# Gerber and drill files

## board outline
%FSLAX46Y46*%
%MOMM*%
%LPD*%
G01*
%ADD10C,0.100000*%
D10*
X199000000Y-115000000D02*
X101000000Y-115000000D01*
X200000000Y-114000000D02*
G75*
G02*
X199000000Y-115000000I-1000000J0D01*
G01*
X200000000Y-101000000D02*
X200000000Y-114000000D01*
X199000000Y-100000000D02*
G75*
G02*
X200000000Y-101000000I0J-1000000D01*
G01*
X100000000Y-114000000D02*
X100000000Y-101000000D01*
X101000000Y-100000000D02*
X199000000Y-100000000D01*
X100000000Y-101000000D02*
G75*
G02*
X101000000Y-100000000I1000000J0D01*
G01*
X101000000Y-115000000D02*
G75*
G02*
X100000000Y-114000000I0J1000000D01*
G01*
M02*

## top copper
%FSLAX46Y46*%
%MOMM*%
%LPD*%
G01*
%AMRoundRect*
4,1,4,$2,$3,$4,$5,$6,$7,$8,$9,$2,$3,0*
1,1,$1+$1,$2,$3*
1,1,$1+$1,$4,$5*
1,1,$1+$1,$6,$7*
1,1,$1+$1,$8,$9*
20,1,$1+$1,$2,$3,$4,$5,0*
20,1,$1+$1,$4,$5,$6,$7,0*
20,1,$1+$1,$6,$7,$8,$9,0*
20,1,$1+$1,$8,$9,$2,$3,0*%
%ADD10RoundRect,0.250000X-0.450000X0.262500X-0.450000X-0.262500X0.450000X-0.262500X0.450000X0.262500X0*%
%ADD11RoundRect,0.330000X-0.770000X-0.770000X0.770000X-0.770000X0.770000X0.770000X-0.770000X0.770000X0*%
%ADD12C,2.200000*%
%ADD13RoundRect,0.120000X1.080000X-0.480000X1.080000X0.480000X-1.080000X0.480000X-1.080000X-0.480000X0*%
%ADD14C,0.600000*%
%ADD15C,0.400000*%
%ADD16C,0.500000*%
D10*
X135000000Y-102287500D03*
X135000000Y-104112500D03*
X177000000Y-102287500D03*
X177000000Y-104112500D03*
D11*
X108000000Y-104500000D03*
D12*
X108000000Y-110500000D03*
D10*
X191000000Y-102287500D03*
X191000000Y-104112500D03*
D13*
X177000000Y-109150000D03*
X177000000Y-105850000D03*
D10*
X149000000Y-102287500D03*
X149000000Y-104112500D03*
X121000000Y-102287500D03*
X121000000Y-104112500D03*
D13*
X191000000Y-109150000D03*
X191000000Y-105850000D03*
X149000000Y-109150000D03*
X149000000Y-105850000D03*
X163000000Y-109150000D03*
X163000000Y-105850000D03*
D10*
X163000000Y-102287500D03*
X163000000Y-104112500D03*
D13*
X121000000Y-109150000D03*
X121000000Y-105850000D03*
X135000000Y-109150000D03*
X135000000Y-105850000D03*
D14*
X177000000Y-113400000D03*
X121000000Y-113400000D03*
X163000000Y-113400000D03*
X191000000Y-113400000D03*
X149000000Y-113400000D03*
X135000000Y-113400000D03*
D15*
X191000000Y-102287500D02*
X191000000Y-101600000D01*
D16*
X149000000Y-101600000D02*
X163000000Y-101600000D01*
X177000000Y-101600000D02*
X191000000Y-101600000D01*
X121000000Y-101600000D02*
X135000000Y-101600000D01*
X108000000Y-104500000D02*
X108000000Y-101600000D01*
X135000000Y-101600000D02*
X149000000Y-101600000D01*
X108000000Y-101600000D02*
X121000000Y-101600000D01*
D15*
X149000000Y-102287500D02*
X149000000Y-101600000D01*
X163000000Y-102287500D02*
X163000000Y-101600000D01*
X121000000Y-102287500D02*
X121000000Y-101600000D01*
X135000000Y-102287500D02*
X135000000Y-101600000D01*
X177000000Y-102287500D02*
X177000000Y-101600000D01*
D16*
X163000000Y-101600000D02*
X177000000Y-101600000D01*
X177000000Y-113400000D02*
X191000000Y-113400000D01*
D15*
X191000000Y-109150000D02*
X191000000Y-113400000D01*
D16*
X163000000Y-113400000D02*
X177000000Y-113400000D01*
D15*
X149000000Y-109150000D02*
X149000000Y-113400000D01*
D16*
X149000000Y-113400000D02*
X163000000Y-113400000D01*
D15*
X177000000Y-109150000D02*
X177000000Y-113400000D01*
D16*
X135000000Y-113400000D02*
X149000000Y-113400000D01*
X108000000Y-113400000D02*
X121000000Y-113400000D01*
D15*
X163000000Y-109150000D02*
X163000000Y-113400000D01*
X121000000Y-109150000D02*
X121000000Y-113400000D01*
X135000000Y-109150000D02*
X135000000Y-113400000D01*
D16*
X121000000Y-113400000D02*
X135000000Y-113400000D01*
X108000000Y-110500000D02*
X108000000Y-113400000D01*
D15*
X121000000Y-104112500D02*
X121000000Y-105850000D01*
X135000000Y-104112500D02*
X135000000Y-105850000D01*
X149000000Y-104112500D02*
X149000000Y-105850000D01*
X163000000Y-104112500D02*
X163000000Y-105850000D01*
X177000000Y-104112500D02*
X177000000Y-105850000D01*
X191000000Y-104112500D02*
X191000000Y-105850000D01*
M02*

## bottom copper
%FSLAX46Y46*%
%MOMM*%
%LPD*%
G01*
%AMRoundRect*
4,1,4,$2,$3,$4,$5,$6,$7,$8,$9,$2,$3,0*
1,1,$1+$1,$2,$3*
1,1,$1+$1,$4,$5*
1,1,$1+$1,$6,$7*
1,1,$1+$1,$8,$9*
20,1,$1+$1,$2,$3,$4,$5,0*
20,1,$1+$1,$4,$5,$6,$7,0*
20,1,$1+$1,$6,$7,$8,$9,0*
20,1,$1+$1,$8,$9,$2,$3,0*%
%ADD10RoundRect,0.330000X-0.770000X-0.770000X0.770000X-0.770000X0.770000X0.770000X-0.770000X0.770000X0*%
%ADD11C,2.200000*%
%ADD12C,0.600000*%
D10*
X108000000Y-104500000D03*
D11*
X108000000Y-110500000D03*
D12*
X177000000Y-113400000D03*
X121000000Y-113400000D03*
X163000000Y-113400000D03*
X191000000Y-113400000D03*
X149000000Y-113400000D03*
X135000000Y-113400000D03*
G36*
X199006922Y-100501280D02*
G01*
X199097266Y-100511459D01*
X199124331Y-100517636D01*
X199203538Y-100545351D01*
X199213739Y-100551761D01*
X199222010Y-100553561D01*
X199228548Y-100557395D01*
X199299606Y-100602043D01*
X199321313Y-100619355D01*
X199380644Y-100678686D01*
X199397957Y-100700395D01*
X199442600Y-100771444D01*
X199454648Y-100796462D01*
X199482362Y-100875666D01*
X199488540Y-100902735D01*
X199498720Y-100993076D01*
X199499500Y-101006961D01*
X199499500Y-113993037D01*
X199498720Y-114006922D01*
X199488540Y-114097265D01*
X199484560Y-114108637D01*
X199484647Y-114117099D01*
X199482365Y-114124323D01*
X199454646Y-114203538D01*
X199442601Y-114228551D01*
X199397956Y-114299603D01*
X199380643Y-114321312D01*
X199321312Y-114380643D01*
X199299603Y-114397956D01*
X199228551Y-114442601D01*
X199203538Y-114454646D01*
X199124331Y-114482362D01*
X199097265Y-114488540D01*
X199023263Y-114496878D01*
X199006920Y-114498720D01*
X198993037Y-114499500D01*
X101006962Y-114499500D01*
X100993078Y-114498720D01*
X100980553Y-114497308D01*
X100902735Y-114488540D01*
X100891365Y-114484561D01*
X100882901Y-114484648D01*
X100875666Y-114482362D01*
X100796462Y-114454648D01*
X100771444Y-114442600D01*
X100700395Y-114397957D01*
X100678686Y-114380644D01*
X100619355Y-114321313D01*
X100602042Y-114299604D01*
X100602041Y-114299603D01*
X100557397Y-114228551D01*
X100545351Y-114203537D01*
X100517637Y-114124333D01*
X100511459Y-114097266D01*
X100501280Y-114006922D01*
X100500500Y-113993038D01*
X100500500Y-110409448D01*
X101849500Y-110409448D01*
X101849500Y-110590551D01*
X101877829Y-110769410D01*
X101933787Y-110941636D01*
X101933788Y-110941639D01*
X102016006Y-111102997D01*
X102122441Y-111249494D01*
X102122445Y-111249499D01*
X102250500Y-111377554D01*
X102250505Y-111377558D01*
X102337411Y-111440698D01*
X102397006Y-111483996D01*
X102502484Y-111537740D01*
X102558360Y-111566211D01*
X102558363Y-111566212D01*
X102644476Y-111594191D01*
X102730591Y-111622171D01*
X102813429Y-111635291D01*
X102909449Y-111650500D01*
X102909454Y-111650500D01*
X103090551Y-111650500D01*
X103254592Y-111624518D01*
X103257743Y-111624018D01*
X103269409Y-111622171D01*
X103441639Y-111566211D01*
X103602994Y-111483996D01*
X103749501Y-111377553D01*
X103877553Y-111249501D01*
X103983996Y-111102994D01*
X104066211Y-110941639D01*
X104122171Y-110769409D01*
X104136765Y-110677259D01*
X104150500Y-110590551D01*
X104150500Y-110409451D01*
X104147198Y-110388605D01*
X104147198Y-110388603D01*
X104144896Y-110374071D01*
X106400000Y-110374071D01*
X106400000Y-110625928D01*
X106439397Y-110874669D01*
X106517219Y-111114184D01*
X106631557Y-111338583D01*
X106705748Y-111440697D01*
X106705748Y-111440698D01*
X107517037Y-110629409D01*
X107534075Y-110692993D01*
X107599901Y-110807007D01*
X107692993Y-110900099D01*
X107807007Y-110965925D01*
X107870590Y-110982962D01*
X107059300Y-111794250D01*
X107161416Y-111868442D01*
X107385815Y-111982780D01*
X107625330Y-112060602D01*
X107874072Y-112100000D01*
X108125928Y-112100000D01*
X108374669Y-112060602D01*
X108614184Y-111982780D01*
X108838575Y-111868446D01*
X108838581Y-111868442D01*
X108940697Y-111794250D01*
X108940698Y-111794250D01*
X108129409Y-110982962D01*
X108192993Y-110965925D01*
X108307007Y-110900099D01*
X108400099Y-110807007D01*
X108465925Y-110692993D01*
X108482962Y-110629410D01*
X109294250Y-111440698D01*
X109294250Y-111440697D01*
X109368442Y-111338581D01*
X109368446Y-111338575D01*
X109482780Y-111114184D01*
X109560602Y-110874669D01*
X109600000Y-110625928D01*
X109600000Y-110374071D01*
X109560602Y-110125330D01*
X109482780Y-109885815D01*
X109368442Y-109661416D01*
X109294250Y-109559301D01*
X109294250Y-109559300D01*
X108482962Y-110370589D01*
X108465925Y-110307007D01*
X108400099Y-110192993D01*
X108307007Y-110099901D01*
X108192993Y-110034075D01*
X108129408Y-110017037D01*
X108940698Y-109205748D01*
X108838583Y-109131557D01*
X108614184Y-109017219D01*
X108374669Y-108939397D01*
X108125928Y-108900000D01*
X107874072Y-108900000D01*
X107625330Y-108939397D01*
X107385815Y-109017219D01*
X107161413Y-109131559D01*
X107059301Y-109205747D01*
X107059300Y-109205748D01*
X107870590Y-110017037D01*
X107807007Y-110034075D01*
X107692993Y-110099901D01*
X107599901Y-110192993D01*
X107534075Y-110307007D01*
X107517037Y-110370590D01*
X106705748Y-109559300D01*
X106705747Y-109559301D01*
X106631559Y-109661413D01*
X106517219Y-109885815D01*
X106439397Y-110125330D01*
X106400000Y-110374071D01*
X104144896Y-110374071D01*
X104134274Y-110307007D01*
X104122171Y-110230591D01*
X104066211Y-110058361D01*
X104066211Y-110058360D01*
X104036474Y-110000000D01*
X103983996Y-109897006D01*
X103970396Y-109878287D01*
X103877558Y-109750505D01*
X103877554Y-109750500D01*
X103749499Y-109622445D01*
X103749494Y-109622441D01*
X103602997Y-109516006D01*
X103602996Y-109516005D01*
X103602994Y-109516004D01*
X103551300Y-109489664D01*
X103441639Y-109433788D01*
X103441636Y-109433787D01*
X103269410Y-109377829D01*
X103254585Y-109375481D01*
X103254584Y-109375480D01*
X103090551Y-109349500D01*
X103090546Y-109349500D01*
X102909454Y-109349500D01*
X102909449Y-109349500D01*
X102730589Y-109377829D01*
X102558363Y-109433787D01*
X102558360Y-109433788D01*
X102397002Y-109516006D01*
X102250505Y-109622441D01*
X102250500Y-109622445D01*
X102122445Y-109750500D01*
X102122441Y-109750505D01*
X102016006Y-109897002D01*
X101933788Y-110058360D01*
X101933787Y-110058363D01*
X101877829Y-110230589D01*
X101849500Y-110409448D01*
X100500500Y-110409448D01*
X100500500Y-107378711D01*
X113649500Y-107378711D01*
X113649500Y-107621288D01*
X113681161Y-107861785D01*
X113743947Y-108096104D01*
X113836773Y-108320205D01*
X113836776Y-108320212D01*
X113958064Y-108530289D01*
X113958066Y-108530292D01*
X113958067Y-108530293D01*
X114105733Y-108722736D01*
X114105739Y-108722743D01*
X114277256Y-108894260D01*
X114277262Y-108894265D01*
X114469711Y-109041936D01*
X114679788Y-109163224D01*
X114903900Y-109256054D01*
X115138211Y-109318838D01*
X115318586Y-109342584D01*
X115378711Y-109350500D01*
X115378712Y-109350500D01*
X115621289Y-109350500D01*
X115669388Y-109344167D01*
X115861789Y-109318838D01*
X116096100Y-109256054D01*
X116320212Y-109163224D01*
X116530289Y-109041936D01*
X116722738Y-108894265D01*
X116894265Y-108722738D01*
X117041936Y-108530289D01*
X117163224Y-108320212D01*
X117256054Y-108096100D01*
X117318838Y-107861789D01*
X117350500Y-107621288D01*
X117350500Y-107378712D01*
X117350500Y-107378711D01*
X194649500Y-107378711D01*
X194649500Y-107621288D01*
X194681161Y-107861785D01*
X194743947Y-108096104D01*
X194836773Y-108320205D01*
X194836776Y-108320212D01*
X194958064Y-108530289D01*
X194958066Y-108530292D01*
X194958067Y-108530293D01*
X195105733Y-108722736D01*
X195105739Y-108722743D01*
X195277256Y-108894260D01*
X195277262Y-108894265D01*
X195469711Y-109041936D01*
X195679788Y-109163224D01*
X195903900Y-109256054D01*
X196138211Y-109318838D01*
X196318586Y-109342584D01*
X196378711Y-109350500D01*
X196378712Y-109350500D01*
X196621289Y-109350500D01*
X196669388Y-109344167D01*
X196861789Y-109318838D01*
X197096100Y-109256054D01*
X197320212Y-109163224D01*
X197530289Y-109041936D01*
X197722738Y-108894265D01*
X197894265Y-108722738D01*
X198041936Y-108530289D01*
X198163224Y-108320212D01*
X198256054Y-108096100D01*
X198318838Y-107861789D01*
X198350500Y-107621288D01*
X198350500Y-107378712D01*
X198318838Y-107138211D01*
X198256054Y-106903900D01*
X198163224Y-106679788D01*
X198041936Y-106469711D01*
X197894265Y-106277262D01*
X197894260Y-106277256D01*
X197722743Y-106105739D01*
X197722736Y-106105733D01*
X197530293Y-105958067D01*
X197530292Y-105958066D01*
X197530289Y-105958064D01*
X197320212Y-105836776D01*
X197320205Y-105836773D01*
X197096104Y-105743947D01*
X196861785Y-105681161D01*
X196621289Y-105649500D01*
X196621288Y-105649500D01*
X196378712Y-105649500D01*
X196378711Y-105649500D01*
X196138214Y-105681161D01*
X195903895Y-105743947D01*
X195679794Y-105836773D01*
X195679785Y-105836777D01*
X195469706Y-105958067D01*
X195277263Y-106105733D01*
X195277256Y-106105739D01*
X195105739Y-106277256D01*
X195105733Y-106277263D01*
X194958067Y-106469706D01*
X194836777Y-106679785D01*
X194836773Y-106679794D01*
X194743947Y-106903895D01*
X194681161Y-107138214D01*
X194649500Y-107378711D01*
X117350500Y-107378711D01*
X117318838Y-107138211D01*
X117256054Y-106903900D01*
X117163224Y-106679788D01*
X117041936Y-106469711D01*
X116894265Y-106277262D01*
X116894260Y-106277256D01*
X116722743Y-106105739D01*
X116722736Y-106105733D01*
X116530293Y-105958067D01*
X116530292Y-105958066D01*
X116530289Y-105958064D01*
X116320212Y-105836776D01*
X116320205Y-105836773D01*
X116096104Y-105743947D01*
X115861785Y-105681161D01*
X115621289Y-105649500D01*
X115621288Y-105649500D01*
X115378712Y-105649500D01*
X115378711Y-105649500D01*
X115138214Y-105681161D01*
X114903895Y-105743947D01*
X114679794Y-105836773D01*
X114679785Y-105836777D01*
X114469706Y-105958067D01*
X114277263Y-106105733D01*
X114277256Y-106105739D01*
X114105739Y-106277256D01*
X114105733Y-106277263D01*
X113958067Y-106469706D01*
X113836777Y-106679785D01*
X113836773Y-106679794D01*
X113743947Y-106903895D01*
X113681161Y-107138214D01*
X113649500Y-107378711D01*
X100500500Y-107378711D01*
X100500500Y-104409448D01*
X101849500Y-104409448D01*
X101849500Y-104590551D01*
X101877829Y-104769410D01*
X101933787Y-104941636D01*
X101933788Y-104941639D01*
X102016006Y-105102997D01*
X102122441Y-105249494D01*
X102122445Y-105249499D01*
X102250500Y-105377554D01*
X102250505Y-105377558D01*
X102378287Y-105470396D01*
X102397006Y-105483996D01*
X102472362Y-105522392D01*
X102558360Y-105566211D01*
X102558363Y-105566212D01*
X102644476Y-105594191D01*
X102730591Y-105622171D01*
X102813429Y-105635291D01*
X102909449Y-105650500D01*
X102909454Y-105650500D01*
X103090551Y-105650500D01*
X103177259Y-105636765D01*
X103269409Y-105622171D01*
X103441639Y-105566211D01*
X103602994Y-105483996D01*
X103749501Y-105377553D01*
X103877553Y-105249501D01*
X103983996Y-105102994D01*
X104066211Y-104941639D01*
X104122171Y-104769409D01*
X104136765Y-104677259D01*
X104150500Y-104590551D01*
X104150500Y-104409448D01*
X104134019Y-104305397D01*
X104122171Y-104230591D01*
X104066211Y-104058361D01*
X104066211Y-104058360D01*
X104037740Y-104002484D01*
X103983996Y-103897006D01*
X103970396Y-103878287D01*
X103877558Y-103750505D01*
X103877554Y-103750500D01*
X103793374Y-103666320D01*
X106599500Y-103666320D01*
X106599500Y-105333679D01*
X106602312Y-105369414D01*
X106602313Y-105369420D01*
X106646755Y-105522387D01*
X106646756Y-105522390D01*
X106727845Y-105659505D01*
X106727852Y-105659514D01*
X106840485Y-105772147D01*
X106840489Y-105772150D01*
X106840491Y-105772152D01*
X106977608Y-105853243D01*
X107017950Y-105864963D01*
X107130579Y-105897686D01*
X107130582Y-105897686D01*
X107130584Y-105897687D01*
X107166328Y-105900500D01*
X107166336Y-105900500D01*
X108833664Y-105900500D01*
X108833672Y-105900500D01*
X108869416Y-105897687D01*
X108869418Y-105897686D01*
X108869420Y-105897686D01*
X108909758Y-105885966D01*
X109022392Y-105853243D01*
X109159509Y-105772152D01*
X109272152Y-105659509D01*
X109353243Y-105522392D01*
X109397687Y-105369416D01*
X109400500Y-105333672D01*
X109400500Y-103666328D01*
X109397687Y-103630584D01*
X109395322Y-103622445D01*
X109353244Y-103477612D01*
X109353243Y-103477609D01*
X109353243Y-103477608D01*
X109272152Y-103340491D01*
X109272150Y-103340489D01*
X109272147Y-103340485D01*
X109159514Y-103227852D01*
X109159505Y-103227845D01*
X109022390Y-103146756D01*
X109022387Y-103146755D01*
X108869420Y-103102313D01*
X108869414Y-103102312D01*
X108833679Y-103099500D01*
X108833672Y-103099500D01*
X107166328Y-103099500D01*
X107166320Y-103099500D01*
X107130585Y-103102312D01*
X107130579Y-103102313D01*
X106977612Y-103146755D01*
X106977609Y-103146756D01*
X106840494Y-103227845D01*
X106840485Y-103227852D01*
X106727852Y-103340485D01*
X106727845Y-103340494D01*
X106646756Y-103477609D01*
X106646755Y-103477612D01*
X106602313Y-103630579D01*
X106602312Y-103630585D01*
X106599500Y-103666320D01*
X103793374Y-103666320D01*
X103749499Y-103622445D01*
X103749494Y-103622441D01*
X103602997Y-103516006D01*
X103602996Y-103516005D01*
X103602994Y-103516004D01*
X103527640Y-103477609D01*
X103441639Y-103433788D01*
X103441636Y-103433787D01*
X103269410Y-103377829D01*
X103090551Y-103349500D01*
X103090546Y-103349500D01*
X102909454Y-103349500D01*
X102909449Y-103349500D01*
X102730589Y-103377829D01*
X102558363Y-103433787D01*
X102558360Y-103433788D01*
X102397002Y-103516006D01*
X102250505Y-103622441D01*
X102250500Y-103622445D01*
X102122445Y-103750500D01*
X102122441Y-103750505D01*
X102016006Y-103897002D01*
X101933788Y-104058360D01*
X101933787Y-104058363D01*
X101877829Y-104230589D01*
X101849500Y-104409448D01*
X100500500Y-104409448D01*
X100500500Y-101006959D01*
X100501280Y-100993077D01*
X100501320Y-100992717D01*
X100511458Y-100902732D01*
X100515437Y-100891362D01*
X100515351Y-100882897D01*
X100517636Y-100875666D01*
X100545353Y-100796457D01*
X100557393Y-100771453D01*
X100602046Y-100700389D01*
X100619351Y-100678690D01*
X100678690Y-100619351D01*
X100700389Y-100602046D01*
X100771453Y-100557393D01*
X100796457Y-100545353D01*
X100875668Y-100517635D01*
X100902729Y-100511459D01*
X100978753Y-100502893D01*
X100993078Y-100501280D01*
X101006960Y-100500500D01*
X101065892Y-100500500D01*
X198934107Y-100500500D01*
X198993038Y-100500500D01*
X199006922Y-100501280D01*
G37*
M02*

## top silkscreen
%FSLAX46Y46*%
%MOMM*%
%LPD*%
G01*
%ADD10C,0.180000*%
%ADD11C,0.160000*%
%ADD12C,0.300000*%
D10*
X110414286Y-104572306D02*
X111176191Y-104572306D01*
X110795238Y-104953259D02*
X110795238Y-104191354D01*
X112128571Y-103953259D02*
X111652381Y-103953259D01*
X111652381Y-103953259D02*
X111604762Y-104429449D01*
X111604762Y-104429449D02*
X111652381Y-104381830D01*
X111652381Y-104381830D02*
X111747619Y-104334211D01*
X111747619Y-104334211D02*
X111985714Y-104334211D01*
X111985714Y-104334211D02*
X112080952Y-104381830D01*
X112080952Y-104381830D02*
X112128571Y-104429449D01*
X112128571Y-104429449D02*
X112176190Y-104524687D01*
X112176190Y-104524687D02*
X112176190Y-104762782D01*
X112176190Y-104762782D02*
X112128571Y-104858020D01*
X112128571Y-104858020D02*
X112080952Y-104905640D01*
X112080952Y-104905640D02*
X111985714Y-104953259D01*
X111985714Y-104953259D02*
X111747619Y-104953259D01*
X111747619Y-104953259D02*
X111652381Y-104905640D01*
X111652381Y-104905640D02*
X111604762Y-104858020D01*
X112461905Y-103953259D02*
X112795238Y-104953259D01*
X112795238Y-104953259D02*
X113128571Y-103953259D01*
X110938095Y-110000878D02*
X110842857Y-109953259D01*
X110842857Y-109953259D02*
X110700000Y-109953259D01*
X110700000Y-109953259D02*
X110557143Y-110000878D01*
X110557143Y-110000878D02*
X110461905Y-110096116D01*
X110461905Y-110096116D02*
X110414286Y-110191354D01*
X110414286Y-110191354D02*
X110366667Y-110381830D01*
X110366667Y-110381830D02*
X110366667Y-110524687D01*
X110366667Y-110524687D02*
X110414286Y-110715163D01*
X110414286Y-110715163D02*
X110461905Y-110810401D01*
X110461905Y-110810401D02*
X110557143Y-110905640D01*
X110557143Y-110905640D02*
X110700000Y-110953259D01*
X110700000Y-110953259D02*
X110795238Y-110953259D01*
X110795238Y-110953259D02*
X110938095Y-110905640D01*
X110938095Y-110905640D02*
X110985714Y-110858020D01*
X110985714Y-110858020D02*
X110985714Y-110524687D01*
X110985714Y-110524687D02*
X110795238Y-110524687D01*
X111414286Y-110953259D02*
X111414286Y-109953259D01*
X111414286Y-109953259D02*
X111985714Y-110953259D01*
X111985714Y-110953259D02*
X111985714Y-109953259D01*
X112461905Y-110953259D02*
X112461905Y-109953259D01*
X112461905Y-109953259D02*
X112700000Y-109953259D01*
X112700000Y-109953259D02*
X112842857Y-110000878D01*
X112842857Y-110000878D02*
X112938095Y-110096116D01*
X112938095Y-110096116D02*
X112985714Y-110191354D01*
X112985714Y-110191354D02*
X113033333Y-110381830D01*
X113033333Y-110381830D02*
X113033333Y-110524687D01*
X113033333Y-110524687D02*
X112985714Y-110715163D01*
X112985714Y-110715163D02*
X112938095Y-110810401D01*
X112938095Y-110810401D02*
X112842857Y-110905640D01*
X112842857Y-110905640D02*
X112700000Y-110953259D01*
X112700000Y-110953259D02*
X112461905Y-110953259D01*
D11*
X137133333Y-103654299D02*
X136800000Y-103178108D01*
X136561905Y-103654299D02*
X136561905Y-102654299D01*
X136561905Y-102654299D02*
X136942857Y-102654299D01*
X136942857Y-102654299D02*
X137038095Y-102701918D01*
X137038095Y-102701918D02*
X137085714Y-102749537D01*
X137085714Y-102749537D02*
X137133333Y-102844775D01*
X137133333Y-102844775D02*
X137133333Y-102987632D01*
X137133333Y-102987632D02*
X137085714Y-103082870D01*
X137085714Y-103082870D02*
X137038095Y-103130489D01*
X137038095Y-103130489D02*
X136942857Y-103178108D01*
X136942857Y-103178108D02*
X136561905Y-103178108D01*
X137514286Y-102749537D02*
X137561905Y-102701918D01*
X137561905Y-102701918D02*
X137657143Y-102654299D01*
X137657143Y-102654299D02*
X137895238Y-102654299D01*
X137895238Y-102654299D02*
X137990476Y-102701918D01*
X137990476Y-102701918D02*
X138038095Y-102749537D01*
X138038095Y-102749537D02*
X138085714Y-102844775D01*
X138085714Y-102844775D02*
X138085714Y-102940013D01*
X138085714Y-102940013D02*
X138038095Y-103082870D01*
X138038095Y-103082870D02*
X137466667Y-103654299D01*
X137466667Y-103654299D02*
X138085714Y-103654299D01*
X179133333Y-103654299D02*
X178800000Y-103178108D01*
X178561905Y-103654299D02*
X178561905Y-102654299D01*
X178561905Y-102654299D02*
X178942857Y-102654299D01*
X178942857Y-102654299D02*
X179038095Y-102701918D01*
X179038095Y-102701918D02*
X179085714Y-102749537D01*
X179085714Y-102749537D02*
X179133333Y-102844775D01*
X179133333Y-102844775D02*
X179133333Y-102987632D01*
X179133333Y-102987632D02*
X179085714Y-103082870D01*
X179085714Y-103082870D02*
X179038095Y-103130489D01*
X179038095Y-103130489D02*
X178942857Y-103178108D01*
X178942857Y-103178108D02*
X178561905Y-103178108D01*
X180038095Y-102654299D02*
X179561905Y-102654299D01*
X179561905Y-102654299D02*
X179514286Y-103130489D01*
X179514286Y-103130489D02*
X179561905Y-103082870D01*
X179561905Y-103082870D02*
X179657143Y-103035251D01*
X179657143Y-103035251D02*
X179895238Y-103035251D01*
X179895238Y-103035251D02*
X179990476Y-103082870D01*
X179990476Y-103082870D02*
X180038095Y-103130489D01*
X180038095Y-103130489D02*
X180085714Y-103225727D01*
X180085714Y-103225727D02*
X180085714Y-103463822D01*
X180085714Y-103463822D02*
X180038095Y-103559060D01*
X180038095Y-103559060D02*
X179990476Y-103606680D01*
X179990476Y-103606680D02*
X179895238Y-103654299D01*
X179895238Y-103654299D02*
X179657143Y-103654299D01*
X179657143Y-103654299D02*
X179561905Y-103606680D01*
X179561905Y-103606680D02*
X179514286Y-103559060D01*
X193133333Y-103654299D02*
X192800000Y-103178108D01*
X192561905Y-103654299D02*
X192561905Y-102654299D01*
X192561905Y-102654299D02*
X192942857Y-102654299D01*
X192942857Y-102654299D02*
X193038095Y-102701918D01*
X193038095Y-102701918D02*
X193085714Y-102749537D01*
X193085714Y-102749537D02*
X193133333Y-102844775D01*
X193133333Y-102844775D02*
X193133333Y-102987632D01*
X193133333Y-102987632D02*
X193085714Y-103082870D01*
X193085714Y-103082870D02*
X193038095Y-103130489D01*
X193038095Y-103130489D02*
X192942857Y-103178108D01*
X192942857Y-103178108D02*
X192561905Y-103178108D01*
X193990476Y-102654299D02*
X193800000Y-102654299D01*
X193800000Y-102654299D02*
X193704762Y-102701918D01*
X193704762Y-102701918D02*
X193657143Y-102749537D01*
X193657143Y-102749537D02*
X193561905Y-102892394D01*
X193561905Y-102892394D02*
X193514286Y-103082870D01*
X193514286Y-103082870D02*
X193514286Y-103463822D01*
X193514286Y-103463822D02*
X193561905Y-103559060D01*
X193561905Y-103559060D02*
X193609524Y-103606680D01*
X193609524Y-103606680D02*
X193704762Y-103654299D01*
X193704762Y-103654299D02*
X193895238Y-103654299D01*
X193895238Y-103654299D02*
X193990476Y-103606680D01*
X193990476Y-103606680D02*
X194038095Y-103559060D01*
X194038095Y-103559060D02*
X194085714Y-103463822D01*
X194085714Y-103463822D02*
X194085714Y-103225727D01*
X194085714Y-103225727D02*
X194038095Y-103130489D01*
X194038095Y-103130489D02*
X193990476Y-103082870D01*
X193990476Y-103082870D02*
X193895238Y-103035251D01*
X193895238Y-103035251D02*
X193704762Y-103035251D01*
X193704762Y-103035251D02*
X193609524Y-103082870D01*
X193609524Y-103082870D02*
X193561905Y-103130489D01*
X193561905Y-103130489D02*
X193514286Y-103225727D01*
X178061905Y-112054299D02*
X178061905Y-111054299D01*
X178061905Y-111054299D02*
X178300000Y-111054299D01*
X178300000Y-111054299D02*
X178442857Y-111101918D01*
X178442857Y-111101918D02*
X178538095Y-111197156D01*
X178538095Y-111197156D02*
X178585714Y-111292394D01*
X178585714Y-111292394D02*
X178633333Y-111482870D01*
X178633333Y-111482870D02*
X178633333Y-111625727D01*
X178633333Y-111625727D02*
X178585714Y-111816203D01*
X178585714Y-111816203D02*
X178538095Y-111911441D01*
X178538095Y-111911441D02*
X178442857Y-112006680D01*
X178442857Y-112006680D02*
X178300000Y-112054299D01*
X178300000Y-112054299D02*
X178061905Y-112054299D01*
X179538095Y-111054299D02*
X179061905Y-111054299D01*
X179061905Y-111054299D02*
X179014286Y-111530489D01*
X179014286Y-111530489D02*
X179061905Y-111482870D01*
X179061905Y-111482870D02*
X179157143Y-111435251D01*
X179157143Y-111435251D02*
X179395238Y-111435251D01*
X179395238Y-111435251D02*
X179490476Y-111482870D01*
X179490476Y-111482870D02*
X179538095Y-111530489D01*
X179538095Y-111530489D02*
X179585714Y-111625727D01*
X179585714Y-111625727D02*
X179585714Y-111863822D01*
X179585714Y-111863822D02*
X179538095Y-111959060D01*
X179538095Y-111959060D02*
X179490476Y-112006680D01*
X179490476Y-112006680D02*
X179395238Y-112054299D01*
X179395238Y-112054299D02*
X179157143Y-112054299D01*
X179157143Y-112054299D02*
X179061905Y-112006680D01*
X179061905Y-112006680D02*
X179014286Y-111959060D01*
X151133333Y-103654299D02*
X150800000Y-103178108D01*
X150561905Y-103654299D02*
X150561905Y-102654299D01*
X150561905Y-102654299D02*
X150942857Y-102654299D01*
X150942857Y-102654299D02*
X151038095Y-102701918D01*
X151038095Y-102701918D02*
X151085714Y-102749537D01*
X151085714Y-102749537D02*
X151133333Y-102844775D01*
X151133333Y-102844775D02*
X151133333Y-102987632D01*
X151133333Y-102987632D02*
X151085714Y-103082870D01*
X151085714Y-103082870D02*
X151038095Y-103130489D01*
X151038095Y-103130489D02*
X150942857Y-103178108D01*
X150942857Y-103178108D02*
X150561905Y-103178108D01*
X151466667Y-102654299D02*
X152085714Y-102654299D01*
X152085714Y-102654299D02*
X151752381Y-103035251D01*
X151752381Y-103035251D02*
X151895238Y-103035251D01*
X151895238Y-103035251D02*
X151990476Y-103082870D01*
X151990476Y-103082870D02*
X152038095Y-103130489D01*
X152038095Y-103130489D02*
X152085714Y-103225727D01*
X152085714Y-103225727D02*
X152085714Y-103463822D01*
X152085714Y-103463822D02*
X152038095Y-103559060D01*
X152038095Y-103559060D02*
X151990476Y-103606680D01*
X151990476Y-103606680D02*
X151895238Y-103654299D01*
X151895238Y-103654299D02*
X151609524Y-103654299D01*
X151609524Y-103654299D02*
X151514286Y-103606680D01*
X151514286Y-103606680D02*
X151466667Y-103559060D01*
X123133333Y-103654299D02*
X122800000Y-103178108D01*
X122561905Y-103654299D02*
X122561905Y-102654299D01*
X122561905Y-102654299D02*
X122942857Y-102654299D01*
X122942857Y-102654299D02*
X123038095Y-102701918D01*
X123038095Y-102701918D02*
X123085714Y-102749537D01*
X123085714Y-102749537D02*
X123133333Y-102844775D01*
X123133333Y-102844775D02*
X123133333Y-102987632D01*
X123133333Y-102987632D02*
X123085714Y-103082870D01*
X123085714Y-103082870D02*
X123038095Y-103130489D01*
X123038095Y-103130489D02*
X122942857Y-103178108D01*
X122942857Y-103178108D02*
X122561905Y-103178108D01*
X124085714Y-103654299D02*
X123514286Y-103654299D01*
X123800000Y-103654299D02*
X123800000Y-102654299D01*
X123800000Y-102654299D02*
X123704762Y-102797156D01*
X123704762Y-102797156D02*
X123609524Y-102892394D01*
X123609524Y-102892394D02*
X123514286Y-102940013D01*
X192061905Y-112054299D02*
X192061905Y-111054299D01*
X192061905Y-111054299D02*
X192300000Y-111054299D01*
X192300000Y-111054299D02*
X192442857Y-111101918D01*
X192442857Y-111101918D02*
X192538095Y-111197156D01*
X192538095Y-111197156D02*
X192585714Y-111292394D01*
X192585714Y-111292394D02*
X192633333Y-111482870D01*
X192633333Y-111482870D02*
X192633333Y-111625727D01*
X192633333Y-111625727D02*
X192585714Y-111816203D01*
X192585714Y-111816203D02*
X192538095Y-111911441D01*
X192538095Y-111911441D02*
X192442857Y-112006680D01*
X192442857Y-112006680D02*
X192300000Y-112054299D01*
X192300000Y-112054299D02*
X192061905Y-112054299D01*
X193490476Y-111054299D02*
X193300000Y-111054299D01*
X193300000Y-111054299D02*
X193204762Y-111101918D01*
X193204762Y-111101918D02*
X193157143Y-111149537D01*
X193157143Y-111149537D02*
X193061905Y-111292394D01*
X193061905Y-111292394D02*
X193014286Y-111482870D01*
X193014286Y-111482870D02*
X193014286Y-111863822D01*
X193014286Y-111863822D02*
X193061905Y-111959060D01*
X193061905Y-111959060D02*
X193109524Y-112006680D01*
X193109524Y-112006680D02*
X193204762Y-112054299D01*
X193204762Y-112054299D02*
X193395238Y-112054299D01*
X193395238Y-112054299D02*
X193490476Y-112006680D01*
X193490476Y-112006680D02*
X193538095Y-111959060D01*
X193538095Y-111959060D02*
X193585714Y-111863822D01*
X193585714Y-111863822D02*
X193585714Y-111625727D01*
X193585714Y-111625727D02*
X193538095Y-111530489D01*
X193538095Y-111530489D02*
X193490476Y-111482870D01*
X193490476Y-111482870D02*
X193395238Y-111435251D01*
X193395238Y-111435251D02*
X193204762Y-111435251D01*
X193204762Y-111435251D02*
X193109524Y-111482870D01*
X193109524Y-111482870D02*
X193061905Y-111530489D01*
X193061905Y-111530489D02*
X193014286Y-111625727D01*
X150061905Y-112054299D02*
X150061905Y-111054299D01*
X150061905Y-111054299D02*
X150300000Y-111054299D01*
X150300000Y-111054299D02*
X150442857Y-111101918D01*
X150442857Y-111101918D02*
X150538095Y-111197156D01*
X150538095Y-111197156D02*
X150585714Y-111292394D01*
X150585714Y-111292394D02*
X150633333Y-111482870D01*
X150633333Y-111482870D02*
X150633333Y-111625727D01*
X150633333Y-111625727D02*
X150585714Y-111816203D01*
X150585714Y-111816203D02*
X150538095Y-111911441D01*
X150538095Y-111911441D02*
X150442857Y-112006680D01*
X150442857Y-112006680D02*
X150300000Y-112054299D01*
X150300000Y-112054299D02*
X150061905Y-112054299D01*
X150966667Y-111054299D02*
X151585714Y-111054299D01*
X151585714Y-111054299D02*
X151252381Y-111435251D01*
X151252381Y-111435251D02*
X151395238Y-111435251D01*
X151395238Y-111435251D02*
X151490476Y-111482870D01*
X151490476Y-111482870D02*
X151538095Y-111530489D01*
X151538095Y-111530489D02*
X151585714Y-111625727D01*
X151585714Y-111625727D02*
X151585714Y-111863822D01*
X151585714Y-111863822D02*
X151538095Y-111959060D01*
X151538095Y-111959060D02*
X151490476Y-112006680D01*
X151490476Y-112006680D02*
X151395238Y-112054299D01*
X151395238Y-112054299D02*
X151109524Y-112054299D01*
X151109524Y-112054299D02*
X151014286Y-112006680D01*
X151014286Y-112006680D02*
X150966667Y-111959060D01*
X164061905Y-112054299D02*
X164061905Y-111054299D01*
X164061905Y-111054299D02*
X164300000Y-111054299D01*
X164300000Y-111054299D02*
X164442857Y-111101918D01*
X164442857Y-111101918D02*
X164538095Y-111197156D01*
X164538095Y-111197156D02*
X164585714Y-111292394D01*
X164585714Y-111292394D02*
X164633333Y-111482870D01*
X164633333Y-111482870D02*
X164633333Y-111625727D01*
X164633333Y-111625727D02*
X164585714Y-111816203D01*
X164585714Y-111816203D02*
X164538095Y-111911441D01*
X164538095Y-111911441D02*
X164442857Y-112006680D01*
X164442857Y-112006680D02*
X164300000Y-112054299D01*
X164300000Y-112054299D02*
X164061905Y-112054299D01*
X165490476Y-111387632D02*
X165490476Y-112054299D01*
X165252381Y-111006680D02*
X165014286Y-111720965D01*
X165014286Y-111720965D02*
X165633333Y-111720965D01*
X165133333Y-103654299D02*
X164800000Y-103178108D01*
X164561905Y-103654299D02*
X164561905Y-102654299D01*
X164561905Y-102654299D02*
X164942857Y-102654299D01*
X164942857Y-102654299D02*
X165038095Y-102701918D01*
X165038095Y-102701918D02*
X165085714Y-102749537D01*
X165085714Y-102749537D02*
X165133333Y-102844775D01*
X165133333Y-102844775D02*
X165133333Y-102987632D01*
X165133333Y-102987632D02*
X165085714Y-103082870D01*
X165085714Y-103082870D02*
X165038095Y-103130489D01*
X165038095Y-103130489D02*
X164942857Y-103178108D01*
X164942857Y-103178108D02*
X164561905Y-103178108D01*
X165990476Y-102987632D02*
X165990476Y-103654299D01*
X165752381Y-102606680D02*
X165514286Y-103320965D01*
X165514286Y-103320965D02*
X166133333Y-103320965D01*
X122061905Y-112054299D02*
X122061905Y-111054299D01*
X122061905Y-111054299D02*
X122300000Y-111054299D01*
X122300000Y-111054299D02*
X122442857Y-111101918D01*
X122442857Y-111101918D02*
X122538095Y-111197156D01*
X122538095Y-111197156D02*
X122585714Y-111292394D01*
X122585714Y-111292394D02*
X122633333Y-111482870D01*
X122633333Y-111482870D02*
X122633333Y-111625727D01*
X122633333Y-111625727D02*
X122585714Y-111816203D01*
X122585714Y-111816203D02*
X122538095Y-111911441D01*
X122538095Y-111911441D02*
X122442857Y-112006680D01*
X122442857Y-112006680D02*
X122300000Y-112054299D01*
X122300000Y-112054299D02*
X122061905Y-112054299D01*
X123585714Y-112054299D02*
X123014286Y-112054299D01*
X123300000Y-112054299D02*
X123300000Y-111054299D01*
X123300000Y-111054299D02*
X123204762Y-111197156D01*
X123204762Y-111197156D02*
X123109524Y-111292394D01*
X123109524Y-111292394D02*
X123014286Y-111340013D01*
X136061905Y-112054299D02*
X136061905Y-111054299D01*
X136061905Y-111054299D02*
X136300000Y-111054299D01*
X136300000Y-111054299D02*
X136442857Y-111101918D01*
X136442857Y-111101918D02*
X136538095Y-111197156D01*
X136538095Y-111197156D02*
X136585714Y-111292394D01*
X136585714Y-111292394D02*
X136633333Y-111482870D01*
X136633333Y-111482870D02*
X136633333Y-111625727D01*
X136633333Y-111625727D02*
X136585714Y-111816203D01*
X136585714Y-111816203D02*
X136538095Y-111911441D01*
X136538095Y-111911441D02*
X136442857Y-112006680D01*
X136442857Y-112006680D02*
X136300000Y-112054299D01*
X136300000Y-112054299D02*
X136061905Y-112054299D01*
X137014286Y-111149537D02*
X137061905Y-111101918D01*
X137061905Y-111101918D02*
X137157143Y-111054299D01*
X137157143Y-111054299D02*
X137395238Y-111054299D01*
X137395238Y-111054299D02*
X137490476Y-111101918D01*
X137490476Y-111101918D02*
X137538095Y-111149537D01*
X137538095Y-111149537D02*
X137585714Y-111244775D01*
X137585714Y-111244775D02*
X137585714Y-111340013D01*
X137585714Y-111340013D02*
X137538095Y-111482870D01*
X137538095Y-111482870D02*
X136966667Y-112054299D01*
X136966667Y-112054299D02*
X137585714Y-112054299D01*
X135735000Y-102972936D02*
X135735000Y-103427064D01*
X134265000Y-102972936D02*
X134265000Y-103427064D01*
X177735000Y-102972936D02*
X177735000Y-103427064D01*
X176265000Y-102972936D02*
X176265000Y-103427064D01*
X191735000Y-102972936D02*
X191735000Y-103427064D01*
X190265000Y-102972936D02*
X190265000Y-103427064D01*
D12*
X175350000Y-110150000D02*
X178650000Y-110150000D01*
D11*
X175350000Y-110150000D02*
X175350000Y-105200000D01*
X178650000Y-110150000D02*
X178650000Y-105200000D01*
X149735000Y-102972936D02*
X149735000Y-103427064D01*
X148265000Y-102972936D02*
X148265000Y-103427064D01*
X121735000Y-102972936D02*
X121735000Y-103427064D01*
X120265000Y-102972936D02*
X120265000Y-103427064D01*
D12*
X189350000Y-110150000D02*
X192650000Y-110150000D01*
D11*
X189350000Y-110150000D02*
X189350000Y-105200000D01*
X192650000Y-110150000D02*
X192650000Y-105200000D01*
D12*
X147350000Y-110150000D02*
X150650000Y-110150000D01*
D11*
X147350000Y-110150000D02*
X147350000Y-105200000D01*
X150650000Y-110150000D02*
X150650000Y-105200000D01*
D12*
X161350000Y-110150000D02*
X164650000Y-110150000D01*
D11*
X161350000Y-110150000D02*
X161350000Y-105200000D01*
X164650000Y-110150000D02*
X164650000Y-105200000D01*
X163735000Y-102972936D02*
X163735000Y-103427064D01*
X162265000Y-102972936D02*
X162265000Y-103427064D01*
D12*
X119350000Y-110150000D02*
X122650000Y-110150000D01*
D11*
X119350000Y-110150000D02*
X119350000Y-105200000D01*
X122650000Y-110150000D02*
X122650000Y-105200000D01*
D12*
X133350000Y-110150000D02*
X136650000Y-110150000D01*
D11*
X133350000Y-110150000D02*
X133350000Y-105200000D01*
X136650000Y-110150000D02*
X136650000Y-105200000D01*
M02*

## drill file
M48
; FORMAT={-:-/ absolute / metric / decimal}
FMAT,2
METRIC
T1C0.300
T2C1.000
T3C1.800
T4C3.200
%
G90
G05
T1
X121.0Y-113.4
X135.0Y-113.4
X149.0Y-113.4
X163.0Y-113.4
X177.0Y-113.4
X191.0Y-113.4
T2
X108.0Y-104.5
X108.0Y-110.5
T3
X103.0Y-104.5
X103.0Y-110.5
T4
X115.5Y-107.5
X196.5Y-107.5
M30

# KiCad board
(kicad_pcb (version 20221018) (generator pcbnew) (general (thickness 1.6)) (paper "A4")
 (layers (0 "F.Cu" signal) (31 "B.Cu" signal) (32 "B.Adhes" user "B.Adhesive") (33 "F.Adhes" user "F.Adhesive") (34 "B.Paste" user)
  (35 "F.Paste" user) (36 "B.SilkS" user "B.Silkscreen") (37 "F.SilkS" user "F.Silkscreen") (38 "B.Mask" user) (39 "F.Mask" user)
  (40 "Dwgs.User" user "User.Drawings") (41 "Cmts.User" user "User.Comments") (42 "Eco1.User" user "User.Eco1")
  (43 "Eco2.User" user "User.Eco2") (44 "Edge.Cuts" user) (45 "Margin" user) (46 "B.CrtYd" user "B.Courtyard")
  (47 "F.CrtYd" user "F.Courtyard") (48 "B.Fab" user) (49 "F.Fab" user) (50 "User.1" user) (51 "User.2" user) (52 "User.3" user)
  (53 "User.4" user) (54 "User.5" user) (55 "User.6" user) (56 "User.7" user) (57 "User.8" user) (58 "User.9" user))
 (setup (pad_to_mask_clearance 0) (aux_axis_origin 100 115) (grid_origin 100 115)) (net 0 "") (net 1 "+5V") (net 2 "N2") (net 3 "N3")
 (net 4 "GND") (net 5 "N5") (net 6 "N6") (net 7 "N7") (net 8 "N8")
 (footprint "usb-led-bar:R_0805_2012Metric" (layer "F.Cu") (at 135 103.2 -90)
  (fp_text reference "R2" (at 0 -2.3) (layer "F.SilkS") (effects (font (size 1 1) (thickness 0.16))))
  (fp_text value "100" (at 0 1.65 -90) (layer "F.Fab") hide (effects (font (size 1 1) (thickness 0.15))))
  (fp_line (start -0.227064 -0.735) (end 0.227064 -0.735) (stroke (width 0.16) (type solid)) (layer "F.SilkS"))
  (fp_line (start -0.227064 0.735) (end 0.227064 0.735) (stroke (width 0.16) (type solid)) (layer "F.SilkS"))
  (pad "1" smd roundrect (at -0.9125 0 270) (size 1.025 1.4) (layers "F.Cu" "F.Paste" "F.Mask") (roundrect_rratio 0.243902) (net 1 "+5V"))
  (pad "2" smd roundrect (at 0.9125 0 270) (size 1.025 1.4) (layers "F.Cu" "F.Paste" "F.Mask") (roundrect_rratio 0.243902) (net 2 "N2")))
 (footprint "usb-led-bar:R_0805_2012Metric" (layer "F.Cu") (at 177 103.2 -90)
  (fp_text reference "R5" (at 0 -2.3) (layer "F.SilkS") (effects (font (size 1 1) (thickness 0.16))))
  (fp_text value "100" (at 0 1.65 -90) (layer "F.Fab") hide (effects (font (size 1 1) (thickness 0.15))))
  (fp_line (start -0.227064 -0.735) (end 0.227064 -0.735) (stroke (width 0.16) (type solid)) (layer "F.SilkS"))
  (fp_line (start -0.227064 0.735) (end 0.227064 0.735) (stroke (width 0.16) (type solid)) (layer "F.SilkS"))
  (pad "1" smd roundrect (at -0.9125 0 270) (size 1.025 1.4) (layers "F.Cu" "F.Paste" "F.Mask") (roundrect_rratio 0.243902) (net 1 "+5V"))
  (pad "2" smd roundrect (at 0.9125 0 270) (size 1.025 1.4) (layers "F.Cu" "F.Paste" "F.Mask") (roundrect_rratio 0.243902) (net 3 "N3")))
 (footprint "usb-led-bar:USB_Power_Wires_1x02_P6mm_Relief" (layer "F.Cu") (at 108 107.5)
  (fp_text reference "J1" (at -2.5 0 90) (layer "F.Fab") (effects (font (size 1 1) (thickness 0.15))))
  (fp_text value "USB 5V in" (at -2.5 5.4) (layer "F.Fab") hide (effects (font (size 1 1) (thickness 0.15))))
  (pad "" np_thru_hole circle (at -5 -3) (size 1.8 1.8) (drill 1.8) (layers "*.Cu" "*.Mask"))
  (pad "" np_thru_hole circle (at -5 3) (size 1.8 1.8) (drill 1.8) (layers "*.Cu" "*.Mask"))
  (pad "1" thru_hole roundrect (at 0 -3) (size 2.2 2.2) (drill 1) (layers "*.Cu" "*.Mask") (roundrect_rratio 0.15) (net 1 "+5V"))
  (pad "2" thru_hole circle (at 0 3) (size 2.2 2.2) (drill 1) (layers "*.Cu" "*.Mask") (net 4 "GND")))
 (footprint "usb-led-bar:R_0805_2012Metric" (layer "F.Cu") (at 191 103.2 -90)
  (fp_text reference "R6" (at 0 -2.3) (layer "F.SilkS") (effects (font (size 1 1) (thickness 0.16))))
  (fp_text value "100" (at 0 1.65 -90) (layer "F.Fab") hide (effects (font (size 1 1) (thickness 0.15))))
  (fp_line (start -0.227064 -0.735) (end 0.227064 -0.735) (stroke (width 0.16) (type solid)) (layer "F.SilkS"))
  (fp_line (start -0.227064 0.735) (end 0.227064 0.735) (stroke (width 0.16) (type solid)) (layer "F.SilkS"))
  (pad "1" smd roundrect (at -0.9125 0 270) (size 1.025 1.4) (layers "F.Cu" "F.Paste" "F.Mask") (roundrect_rratio 0.243902) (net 1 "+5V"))
  (pad "2" smd roundrect (at 0.9125 0 270) (size 1.025 1.4) (layers "F.Cu" "F.Paste" "F.Mask") (roundrect_rratio 0.243902) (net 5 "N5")))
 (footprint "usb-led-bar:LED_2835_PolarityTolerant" (layer "F.Cu") (at 177 107.5 90)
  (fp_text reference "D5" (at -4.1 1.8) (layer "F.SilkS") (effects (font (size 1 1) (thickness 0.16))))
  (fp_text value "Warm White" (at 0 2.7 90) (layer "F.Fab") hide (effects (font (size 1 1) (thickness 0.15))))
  (fp_line (start -2.65 -1.65) (end -2.65 1.65) (stroke (width 0.3) (type solid)) (layer "F.SilkS"))
  (fp_line (start -2.65 -1.65) (end 2.3 -1.65) (stroke (width 0.16) (type solid)) (layer "F.SilkS"))
  (fp_line (start -2.65 1.65) (end 2.3 1.65) (stroke (width 0.16) (type solid)) (layer "F.SilkS"))
  (pad "1" smd roundrect (at -1.65 0 90) (size 1.2 2.4) (layers "F.Cu" "F.Paste" "F.Mask") (roundrect_rratio 0.1) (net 4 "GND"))
  (pad "2" smd roundrect (at 1.65 0 90) (size 1.2 2.4) (layers "F.Cu" "F.Paste" "F.Mask") (roundrect_rratio 0.1) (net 3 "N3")))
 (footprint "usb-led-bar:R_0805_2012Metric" (layer "F.Cu") (at 149 103.2 -90)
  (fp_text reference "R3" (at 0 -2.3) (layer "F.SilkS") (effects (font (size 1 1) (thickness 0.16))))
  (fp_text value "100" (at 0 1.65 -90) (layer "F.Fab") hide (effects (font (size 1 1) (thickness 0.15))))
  (fp_line (start -0.227064 -0.735) (end 0.227064 -0.735) (stroke (width 0.16) (type solid)) (layer "F.SilkS"))
  (fp_line (start -0.227064 0.735) (end 0.227064 0.735) (stroke (width 0.16) (type solid)) (layer "F.SilkS"))
  (pad "1" smd roundrect (at -0.9125 0 270) (size 1.025 1.4) (layers "F.Cu" "F.Paste" "F.Mask") (roundrect_rratio 0.243902) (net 1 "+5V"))
  (pad "2" smd roundrect (at 0.9125 0 270) (size 1.025 1.4) (layers "F.Cu" "F.Paste" "F.Mask") (roundrect_rratio 0.243902) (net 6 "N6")))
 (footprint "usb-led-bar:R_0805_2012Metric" (layer "F.Cu") (at 121 103.2 -90)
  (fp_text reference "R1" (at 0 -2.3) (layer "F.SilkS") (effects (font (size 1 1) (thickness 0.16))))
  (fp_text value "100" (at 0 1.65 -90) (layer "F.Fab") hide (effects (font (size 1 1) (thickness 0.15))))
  (fp_line (start -0.227064 -0.735) (end 0.227064 -0.735) (stroke (width 0.16) (type solid)) (layer "F.SilkS"))
  (fp_line (start -0.227064 0.735) (end 0.227064 0.735) (stroke (width 0.16) (type solid)) (layer "F.SilkS"))
  (pad "1" smd roundrect (at -0.9125 0 270) (size 1.025 1.4) (layers "F.Cu" "F.Paste" "F.Mask") (roundrect_rratio 0.243902) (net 1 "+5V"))
  (pad "2" smd roundrect (at 0.9125 0 270) (size 1.025 1.4) (layers "F.Cu" "F.Paste" "F.Mask") (roundrect_rratio 0.243902) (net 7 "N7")))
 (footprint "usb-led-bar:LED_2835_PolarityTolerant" (layer "F.Cu") (at 191 107.5 90)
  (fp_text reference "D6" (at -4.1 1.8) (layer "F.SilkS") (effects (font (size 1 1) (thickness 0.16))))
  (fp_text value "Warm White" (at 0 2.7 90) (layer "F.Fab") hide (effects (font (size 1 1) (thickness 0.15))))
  (fp_line (start -2.65 -1.65) (end -2.65 1.65) (stroke (width 0.3) (type solid)) (layer "F.SilkS"))
  (fp_line (start -2.65 -1.65) (end 2.3 -1.65) (stroke (width 0.16) (type solid)) (layer "F.SilkS"))
  (fp_line (start -2.65 1.65) (end 2.3 1.65) (stroke (width 0.16) (type solid)) (layer "F.SilkS"))
  (pad "1" smd roundrect (at -1.65 0 90) (size 1.2 2.4) (layers "F.Cu" "F.Paste" "F.Mask") (roundrect_rratio 0.1) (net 4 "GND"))
  (pad "2" smd roundrect (at 1.65 0 90) (size 1.2 2.4) (layers "F.Cu" "F.Paste" "F.Mask") (roundrect_rratio 0.1) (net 5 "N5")))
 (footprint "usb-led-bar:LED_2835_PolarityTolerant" (layer "F.Cu") (at 149 107.5 90)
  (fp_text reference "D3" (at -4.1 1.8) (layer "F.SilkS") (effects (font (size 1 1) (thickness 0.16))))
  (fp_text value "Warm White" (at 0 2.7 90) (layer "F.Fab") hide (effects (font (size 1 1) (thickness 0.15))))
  (fp_line (start -2.65 -1.65) (end -2.65 1.65) (stroke (width 0.3) (type solid)) (layer "F.SilkS"))
  (fp_line (start -2.65 -1.65) (end 2.3 -1.65) (stroke (width 0.16) (type solid)) (layer "F.SilkS"))
  (fp_line (start -2.65 1.65) (end 2.3 1.65) (stroke (width 0.16) (type solid)) (layer "F.SilkS"))
  (pad "1" smd roundrect (at -1.65 0 90) (size 1.2 2.4) (layers "F.Cu" "F.Paste" "F.Mask") (roundrect_rratio 0.1) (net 4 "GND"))
  (pad "2" smd roundrect (at 1.65 0 90) (size 1.2 2.4) (layers "F.Cu" "F.Paste" "F.Mask") (roundrect_rratio 0.1) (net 6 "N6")))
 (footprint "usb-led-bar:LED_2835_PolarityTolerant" (layer "F.Cu") (at 163 107.5 90)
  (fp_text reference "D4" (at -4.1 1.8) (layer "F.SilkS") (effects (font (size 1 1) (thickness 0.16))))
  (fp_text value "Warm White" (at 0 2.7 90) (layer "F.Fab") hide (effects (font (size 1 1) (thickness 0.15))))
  (fp_line (start -2.65 -1.65) (end -2.65 1.65) (stroke (width 0.3) (type solid)) (layer "F.SilkS"))
  (fp_line (start -2.65 -1.65) (end 2.3 -1.65) (stroke (width 0.16) (type solid)) (layer "F.SilkS"))
  (fp_line (start -2.65 1.65) (end 2.3 1.65) (stroke (width 0.16) (type solid)) (layer "F.SilkS"))
  (pad "1" smd roundrect (at -1.65 0 90) (size 1.2 2.4) (layers "F.Cu" "F.Paste" "F.Mask") (roundrect_rratio 0.1) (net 4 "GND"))
  (pad "2" smd roundrect (at 1.65 0 90) (size 1.2 2.4) (layers "F.Cu" "F.Paste" "F.Mask") (roundrect_rratio 0.1) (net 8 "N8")))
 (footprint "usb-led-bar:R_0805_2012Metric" (layer "F.Cu") (at 163 103.2 -90)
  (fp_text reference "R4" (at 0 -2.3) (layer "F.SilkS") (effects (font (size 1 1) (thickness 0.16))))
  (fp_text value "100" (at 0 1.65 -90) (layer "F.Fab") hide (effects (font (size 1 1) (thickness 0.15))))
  (fp_line (start -0.227064 -0.735) (end 0.227064 -0.735) (stroke (width 0.16) (type solid)) (layer "F.SilkS"))
  (fp_line (start -0.227064 0.735) (end 0.227064 0.735) (stroke (width 0.16) (type solid)) (layer "F.SilkS"))
  (pad "1" smd roundrect (at -0.9125 0 270) (size 1.025 1.4) (layers "F.Cu" "F.Paste" "F.Mask") (roundrect_rratio 0.243902) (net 1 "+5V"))
  (pad "2" smd roundrect (at 0.9125 0 270) (size 1.025 1.4) (layers "F.Cu" "F.Paste" "F.Mask") (roundrect_rratio 0.243902) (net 8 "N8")))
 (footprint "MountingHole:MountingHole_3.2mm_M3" (layer "F.Cu") (at 196.5 107.5)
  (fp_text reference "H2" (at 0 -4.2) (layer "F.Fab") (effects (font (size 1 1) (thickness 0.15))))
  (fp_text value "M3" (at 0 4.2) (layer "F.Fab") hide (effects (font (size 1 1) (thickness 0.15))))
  (pad "" np_thru_hole circle (at 0 0) (size 3.2 3.2) (drill 3.2) (layers "*.Cu" "*.Mask")))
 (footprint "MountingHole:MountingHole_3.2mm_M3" (layer "F.Cu") (at 115.5 107.5)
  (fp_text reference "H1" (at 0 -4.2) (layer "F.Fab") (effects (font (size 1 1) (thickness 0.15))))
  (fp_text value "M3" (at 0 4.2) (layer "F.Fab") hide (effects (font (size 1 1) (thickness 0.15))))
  (pad "" np_thru_hole circle (at 0 0) (size 3.2 3.2) (drill 3.2) (layers "*.Cu" "*.Mask")))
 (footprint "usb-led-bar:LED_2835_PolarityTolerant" (layer "F.Cu") (at 121 107.5 90)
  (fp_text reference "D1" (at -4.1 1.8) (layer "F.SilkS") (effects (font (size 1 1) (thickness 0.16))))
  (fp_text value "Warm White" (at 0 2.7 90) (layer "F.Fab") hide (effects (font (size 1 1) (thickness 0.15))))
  (fp_line (start -2.65 -1.65) (end -2.65 1.65) (stroke (width 0.3) (type solid)) (layer "F.SilkS"))
  (fp_line (start -2.65 -1.65) (end 2.3 -1.65) (stroke (width 0.16) (type solid)) (layer "F.SilkS"))
  (fp_line (start -2.65 1.65) (end 2.3 1.65) (stroke (width 0.16) (type solid)) (layer "F.SilkS"))
  (pad "1" smd roundrect (at -1.65 0 90) (size 1.2 2.4) (layers "F.Cu" "F.Paste" "F.Mask") (roundrect_rratio 0.1) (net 4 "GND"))
  (pad "2" smd roundrect (at 1.65 0 90) (size 1.2 2.4) (layers "F.Cu" "F.Paste" "F.Mask") (roundrect_rratio 0.1) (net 7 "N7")))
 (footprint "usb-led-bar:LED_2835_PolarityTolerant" (layer "F.Cu") (at 135 107.5 90)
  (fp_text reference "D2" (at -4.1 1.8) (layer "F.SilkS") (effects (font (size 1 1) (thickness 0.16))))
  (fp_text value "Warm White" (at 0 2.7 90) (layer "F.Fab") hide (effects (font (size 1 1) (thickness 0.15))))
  (fp_line (start -2.65 -1.65) (end -2.65 1.65) (stroke (width 0.3) (type solid)) (layer "F.SilkS"))
  (fp_line (start -2.65 -1.65) (end 2.3 -1.65) (stroke (width 0.16) (type solid)) (layer "F.SilkS"))
  (fp_line (start -2.65 1.65) (end 2.3 1.65) (stroke (width 0.16) (type solid)) (layer "F.SilkS"))
  (pad "1" smd roundrect (at -1.65 0 90) (size 1.2 2.4) (layers "F.Cu" "F.Paste" "F.Mask") (roundrect_rratio 0.1) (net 4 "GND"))
  (pad "2" smd roundrect (at 1.65 0 90) (size 1.2 2.4) (layers "F.Cu" "F.Paste" "F.Mask") (roundrect_rratio 0.1) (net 2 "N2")))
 (gr_line (start 199 115) (end 101 115) (stroke (width 0.1) (type default)) (layer "Edge.Cuts"))
 (gr_arc (start 200 114) (mid 199.707106 114.707106) (end 199 115) (stroke (width 0.1) (type default)) (layer "Edge.Cuts"))
 (gr_line (start 200 101) (end 200 114) (stroke (width 0.1) (type default)) (layer "Edge.Cuts"))
 (gr_arc (start 199 100) (mid 199.707106 100.292893) (end 200 101) (stroke (width 0.1) (type default)) (layer "Edge.Cuts"))
 (gr_line (start 100 114) (end 100 101) (stroke (width 0.1) (type default)) (layer "Edge.Cuts"))
 (gr_line (start 101 100) (end 199 100) (stroke (width 0.1) (type default)) (layer "Edge.Cuts"))
 (gr_arc (start 100 101) (mid 100.292893 100.292893) (end 101 100) (stroke (width 0.1) (type default)) (layer "Edge.Cuts"))
 (gr_arc (start 101 115) (mid 100.292893 114.707106) (end 100 114) (stroke (width 0.1) (type default)) (layer "Edge.Cuts"))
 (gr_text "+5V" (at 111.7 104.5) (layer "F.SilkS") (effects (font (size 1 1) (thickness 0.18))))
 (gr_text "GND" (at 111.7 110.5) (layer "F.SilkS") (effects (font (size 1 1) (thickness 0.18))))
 (segment (start 191 102.2875) (end 191 101.6) (width 0.4) (layer "F.Cu") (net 1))
 (segment (start 149 101.6) (end 163 101.6) (width 0.5) (layer "F.Cu") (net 1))
 (segment (start 177 101.6) (end 191 101.6) (width 0.5) (layer "F.Cu") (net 1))
 (segment (start 121 101.6) (end 135 101.6) (width 0.5) (layer "F.Cu") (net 1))
 (segment (start 108 104.5) (end 108 101.6) (width 0.5) (layer "F.Cu") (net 1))
 (segment (start 135 101.6) (end 149 101.6) (width 0.5) (layer "F.Cu") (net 1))
 (segment (start 108 101.6) (end 121 101.6) (width 0.5) (layer "F.Cu") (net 1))
 (segment (start 149 102.2875) (end 149 101.6) (width 0.4) (layer "F.Cu") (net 1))
 (segment (start 163 102.2875) (end 163 101.6) (width 0.4) (layer "F.Cu") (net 1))
 (segment (start 121 102.2875) (end 121 101.6) (width 0.4) (layer "F.Cu") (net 1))
 (segment (start 135 102.2875) (end 135 101.6) (width 0.4) (layer "F.Cu") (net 1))
 (segment (start 177 102.2875) (end 177 101.6) (width 0.4) (layer "F.Cu") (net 1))
 (segment (start 163 101.6) (end 177 101.6) (width 0.5) (layer "F.Cu") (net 1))
 (segment (start 177 113.4) (end 191 113.4) (width 0.5) (layer "F.Cu") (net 4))
 (segment (start 191 109.15) (end 191 113.4) (width 0.4) (layer "F.Cu") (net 4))
 (segment (start 163 113.4) (end 177 113.4) (width 0.5) (layer "F.Cu") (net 4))
 (segment (start 149 109.15) (end 149 113.4) (width 0.4) (layer "F.Cu") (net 4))
 (segment (start 149 113.4) (end 163 113.4) (width 0.5) (layer "F.Cu") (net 4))
 (segment (start 177 109.15) (end 177 113.4) (width 0.4) (layer "F.Cu") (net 4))
 (segment (start 135 113.4) (end 149 113.4) (width 0.5) (layer "F.Cu") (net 4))
 (segment (start 108 113.4) (end 121 113.4) (width 0.5) (layer "F.Cu") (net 4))
 (segment (start 163 109.15) (end 163 113.4) (width 0.4) (layer "F.Cu") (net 4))
 (segment (start 121 109.15) (end 121 113.4) (width 0.4) (layer "F.Cu") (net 4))
 (segment (start 135 109.15) (end 135 113.4) (width 0.4) (layer "F.Cu") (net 4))
 (segment (start 121 113.4) (end 135 113.4) (width 0.5) (layer "F.Cu") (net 4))
 (segment (start 108 110.5) (end 108 113.4) (width 0.5) (layer "F.Cu") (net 4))
 (via (at 177 113.4) (size 0.6) (drill 0.3) (layers "F.Cu" "B.Cu") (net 4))
 (via (at 121 113.4) (size 0.6) (drill 0.3) (layers "F.Cu" "B.Cu") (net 4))
 (via (at 163 113.4) (size 0.6) (drill 0.3) (layers "F.Cu" "B.Cu") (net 4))
 (via (at 191 113.4) (size 0.6) (drill 0.3) (layers "F.Cu" "B.Cu") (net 4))
 (via (at 149 113.4) (size 0.6) (drill 0.3) (layers "F.Cu" "B.Cu") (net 4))
 (via (at 135 113.4) (size 0.6) (drill 0.3) (layers "F.Cu" "B.Cu") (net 4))
 (segment (start 121 104.1125) (end 121 105.85) (width 0.4) (layer "F.Cu") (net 7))
 (segment (start 135 104.1125) (end 135 105.85) (width 0.4) (layer "F.Cu") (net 2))
 (segment (start 149 104.1125) (end 149 105.85) (width 0.4) (layer "F.Cu") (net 6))
 (segment (start 163 104.1125) (end 163 105.85) (width 0.4) (layer "F.Cu") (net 8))
 (segment (start 177 104.1125) (end 177 105.85) (width 0.4) (layer "F.Cu") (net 3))
 (segment (start 191 104.1125) (end 191 105.85) (width 0.4) (layer "F.Cu") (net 5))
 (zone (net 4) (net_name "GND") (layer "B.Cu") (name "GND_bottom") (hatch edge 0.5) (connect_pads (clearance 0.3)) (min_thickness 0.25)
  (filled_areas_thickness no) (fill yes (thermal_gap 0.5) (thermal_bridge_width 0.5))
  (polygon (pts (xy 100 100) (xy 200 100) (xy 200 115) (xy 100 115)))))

